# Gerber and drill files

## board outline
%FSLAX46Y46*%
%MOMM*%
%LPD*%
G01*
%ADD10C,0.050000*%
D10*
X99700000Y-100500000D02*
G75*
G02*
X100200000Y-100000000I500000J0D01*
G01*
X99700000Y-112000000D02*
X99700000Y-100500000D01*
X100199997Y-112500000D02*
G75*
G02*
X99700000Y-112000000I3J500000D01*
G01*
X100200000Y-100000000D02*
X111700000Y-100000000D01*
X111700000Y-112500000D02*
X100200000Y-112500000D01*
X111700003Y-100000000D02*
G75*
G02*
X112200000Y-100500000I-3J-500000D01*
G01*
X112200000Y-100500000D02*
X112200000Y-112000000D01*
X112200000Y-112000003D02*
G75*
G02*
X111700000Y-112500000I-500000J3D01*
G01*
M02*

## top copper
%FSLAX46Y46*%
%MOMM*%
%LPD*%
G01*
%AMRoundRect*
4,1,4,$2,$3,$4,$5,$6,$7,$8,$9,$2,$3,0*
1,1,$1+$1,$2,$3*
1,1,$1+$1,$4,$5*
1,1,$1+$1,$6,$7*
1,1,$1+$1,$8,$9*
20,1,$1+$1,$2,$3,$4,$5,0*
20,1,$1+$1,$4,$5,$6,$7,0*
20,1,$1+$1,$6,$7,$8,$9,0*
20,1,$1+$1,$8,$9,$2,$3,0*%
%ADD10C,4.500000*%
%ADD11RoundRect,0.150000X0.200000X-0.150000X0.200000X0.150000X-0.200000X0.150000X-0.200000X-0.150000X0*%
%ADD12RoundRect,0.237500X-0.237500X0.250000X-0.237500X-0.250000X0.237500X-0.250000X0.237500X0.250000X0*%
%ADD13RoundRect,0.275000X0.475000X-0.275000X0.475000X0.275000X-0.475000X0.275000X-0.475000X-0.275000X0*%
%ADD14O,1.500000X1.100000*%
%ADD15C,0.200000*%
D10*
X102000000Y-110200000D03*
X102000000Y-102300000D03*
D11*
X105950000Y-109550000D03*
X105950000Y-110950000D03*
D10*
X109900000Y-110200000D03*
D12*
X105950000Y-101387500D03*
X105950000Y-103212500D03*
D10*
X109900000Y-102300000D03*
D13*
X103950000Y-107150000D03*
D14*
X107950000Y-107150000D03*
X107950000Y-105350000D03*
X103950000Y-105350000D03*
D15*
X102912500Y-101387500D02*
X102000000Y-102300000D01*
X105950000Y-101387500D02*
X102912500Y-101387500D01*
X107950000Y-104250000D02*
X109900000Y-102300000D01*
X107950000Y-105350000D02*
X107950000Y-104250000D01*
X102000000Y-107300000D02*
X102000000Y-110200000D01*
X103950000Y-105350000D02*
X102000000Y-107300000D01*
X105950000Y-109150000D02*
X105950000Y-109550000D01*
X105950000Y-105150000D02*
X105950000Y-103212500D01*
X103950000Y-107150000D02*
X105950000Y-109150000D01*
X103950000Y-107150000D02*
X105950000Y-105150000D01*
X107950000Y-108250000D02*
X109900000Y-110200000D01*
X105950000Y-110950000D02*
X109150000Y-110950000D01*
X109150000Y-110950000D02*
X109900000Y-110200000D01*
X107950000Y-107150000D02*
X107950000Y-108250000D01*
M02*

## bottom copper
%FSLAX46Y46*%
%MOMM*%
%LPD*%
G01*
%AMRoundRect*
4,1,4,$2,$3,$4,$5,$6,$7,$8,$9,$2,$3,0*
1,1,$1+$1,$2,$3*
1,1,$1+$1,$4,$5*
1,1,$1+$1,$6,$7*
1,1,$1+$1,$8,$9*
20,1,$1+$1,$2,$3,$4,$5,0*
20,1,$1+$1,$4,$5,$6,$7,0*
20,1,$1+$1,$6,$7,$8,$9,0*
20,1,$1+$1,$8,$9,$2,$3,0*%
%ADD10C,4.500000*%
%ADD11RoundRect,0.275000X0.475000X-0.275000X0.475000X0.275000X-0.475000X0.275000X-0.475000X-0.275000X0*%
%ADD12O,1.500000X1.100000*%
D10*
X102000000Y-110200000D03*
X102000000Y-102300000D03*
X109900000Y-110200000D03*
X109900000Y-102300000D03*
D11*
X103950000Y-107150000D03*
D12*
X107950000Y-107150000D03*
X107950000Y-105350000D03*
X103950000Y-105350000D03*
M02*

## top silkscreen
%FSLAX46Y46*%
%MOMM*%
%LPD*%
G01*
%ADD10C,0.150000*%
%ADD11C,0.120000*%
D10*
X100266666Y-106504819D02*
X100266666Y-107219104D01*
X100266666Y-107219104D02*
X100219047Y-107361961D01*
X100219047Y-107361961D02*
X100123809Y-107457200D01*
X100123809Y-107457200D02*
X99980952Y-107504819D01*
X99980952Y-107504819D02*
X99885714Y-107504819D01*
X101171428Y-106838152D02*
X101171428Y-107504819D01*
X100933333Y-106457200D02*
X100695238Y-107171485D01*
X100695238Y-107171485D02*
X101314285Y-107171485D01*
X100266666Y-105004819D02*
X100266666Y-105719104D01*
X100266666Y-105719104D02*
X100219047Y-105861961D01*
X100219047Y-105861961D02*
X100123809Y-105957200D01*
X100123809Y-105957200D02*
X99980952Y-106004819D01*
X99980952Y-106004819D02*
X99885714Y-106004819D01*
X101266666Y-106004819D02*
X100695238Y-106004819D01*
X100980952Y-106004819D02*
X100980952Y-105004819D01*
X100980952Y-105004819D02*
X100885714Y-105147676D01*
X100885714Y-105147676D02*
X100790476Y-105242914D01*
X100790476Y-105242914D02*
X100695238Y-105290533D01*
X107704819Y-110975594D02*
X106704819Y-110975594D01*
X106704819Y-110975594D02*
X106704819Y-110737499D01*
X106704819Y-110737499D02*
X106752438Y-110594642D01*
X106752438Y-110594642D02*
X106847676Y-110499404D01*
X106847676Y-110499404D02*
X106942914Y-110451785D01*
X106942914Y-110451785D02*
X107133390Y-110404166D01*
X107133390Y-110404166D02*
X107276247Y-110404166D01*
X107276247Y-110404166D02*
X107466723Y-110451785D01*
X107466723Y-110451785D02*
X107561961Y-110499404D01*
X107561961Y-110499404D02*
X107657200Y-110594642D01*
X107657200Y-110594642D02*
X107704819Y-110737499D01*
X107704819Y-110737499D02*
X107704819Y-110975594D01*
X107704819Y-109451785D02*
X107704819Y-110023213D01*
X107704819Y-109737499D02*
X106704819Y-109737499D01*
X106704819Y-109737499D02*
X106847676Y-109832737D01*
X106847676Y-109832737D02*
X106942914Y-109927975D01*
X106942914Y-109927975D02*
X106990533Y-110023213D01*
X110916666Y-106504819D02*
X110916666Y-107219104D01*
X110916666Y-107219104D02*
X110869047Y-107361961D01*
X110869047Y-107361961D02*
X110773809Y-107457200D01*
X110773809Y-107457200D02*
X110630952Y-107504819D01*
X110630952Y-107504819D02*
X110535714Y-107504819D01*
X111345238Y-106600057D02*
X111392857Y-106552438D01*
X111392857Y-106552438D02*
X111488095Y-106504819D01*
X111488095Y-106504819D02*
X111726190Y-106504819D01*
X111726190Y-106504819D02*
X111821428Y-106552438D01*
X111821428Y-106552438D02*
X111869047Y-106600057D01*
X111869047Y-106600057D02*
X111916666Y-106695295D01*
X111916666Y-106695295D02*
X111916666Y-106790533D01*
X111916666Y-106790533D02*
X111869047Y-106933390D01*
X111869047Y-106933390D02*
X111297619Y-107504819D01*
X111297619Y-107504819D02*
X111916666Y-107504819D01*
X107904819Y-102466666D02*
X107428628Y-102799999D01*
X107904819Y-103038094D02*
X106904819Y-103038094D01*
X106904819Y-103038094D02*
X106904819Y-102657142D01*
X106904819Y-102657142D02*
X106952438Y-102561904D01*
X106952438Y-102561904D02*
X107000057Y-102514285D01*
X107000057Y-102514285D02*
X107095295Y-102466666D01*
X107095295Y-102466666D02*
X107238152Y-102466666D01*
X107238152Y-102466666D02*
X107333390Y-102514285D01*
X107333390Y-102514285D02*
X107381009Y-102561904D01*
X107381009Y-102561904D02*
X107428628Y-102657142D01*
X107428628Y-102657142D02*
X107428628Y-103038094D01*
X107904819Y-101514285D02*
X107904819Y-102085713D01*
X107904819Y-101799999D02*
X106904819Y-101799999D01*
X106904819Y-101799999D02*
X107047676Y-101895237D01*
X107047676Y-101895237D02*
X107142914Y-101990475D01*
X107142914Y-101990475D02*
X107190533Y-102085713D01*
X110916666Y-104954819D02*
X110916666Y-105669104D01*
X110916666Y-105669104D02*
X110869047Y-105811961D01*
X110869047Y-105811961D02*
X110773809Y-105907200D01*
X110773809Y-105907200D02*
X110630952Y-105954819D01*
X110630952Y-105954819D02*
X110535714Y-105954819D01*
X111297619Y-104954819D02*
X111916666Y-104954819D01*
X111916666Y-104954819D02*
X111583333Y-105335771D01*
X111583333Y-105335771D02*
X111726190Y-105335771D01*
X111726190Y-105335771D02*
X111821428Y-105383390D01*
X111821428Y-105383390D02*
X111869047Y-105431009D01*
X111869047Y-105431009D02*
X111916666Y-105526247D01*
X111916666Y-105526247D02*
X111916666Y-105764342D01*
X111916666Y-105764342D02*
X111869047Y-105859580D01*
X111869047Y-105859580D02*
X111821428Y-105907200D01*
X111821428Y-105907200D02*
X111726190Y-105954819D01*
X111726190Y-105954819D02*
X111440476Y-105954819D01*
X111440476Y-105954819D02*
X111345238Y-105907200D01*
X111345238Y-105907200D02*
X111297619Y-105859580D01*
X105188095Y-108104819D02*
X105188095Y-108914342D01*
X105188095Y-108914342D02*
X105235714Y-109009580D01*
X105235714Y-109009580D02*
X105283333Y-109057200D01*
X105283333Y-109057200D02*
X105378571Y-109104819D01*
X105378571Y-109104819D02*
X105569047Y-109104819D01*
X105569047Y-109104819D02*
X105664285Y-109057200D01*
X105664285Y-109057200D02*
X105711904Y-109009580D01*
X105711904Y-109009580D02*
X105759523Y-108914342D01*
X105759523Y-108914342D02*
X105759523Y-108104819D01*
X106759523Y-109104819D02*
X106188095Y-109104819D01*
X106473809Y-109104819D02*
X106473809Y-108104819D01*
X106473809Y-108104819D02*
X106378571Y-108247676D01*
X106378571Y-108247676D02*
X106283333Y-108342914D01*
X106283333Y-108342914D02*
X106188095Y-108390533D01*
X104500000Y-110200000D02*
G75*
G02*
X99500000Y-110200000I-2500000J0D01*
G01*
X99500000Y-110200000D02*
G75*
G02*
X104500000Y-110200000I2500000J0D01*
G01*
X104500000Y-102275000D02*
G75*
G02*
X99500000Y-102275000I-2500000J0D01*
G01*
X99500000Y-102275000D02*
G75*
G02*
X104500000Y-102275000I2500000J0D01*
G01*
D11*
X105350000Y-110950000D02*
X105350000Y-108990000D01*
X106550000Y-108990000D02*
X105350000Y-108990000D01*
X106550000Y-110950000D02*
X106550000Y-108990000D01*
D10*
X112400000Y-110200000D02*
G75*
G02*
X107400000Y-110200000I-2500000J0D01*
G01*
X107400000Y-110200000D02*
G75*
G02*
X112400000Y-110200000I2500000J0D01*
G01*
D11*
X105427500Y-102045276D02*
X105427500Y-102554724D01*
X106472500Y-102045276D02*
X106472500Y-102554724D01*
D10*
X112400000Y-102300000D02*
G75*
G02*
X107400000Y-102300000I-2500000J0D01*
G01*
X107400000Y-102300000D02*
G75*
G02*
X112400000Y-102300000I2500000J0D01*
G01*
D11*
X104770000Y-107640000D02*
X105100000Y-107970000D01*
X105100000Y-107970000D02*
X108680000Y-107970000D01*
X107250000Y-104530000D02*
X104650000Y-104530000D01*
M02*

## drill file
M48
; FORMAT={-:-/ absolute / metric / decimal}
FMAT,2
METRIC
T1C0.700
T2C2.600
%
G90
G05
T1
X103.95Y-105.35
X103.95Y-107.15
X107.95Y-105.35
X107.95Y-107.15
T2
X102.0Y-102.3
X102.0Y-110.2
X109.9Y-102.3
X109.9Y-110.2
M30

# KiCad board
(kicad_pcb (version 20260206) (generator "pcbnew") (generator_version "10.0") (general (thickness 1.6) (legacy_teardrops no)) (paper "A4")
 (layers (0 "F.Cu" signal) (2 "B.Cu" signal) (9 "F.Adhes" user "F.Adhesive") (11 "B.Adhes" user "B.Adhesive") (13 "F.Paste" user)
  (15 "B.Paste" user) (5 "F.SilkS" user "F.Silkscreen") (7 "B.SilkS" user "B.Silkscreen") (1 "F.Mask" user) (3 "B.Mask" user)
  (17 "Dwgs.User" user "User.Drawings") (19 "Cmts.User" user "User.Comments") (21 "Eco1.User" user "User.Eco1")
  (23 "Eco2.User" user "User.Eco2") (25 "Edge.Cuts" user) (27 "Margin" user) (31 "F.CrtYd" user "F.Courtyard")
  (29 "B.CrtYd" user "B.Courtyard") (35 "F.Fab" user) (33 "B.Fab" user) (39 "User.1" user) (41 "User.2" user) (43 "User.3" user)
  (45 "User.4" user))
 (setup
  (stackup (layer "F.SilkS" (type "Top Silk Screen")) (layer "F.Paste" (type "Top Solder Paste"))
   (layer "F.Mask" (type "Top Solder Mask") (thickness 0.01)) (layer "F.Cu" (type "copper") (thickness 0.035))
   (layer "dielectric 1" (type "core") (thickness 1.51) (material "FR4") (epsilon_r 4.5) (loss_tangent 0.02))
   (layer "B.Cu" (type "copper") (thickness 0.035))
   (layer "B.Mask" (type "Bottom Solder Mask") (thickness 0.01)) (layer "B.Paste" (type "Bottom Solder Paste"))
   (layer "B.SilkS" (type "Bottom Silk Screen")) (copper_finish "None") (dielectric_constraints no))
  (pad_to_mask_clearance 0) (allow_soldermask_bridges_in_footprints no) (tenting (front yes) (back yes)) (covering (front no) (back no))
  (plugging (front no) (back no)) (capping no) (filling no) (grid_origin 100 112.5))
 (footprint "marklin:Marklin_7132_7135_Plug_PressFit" (layer "F.Cu") (at 102 110.2)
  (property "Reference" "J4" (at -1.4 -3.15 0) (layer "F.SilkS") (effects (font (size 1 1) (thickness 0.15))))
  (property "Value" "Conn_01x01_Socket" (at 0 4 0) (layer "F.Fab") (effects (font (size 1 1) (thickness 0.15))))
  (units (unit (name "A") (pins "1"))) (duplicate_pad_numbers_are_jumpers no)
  (fp_circle (center 0 0) (end 2.5 0) (stroke (width 0.15) (type solid)) (fill no) (layer "F.SilkS"))
  (pad "1" thru_hole circle (at 0 0) (size 4.5 4.5) (drill 2.6) (layers "*.Cu" "*.Mask") (remove_unused_layers no) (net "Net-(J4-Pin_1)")))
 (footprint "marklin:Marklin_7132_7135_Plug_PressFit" (layer "F.Cu") (at 102 102.275)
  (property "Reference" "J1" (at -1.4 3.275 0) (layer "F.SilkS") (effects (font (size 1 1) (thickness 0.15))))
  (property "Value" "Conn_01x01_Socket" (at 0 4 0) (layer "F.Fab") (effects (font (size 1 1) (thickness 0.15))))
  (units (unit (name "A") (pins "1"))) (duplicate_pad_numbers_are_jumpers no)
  (fp_circle (center 0 0) (end 2.5 0) (stroke (width 0.15) (type solid)) (fill no) (layer "F.SilkS"))
  (pad "1" thru_hole circle (at 0 0.025) (size 4.5 4.5) (drill 2.6) (layers "*.Cu" "*.Mask") (remove_unused_layers no)
   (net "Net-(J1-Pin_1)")))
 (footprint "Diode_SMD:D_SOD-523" (layer "F.Cu") (at 105.95 110.25 -90)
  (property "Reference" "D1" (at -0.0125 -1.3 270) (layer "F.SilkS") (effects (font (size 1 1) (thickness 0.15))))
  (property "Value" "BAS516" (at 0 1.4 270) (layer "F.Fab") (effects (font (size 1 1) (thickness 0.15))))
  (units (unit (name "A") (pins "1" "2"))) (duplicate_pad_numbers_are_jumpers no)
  (fp_line (start 0.7 0.6) (end -1.26 0.6) (stroke (width 0.12) (type solid)) (layer "F.SilkS"))
  (fp_line (start -1.26 -0.6) (end -1.26 0.6) (stroke (width 0.12) (type solid)) (layer "F.SilkS"))
  (fp_line (start 0.7 -0.6) (end -1.26 -0.6) (stroke (width 0.12) (type solid)) (layer "F.SilkS"))
  (pad "1" smd roundrect (at -0.7 0 90) (size 0.6 0.7) (layers "F.Cu" "F.Mask" "F.Paste") (roundrect_rratio 0.25) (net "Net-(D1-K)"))
  (pad "2" smd roundrect (at 0.7 0 90) (size 0.6 0.7) (layers "F.Cu" "F.Mask" "F.Paste") (roundrect_rratio 0.25) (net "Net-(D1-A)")))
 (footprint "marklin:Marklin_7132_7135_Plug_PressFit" (layer "F.Cu") (at 109.9 110.2 -90)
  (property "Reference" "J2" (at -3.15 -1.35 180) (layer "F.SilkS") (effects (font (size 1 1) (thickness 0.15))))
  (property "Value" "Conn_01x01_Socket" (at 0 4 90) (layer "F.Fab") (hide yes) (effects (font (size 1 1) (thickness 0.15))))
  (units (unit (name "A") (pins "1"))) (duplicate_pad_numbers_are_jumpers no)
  (fp_circle (center 0 0) (end 2.5 0) (stroke (width 0.15) (type solid)) (fill no) (layer "F.SilkS"))
  (pad "1" thru_hole circle (at 0 0 270) (size 4.5 4.5) (drill 2.6) (layers "*.Cu" "*.Mask") (remove_unused_layers no) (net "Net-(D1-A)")))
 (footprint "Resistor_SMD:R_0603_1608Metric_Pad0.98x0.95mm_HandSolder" (layer "F.Cu") (at 105.95 102.3 -90)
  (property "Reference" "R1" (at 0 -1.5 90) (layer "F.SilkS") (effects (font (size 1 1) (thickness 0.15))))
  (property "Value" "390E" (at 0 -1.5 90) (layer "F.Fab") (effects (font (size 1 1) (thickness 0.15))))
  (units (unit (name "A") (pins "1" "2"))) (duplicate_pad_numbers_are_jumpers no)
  (fp_line (start -0.254724 0.5225) (end 0.254724 0.5225) (stroke (width 0.12) (type solid)) (layer "F.SilkS"))
  (fp_line (start -0.254724 -0.5225) (end 0.254724 -0.5225) (stroke (width 0.12) (type solid)) (layer "F.SilkS"))
  (pad "1" smd roundrect (at -0.9125 0 270) (size 0.975 0.95) (layers "F.Cu" "F.Mask" "F.Paste") (roundrect_rratio 0.25)
   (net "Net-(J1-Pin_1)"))
  (pad "2" smd roundrect (at 0.9125 0 270) (size 0.975 0.95) (layers "F.Cu" "F.Mask" "F.Paste") (roundrect_rratio 0.25) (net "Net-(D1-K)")))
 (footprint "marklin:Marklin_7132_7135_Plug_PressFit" (layer "F.Cu") (at 109.9 102.3)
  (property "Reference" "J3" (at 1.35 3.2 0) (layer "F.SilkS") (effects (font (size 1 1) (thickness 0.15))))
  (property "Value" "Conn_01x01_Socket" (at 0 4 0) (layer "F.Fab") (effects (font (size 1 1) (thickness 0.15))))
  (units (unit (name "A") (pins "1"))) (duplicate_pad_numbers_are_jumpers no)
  (fp_circle (center 0 0) (end 2.5 0) (stroke (width 0.15) (type solid)) (fill no) (layer "F.SilkS"))
  (pad "1" thru_hole circle (at 0 0) (size 4.5 4.5) (drill 2.6) (layers "*.Cu" "*.Mask") (remove_unused_layers no) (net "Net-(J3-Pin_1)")))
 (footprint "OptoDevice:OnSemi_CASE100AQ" (layer "F.Cu") (at 103.95 107.15 90)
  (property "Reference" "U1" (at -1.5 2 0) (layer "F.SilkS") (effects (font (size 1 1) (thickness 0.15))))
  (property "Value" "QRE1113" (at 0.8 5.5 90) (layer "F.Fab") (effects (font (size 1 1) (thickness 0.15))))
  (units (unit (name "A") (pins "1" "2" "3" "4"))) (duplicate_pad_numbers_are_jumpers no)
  (fp_line (start -0.49 0.82) (end -0.82 1.15) (stroke (width 0.12) (type solid)) (layer "F.SilkS"))
  (fp_line (start -0.82 1.15) (end -0.82 4.73) (stroke (width 0.12) (type solid)) (layer "F.SilkS"))
  (fp_line (start 2.62 3.3) (end 2.62 0.7) (stroke (width 0.12) (type solid)) (layer "F.SilkS"))
  (pad "1" thru_hole roundrect (at 0 0 90) (size 1.1 1.5) (drill 0.7) (layers "*.Cu" "*.Mask") (remove_unused_layers no)
   (roundrect_rratio 0.25) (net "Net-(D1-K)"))
  (pad "2" thru_hole oval (at 0 4 90) (size 1.1 1.5) (drill 0.7) (layers "*.Cu" "*.Mask") (remove_unused_layers no) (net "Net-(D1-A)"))
  (pad "3" thru_hole oval (at 1.8 4 90) (size 1.1 1.5) (drill 0.7) (layers "*.Cu" "*.Mask") (remove_unused_layers no) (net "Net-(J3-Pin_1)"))
  (pad "4" thru_hole oval (at 1.8 0 90) (size 1.1 1.5) (drill 0.7) (layers "*.Cu" "*.Mask") (remove_unused_layers no) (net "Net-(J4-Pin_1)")))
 (gr_arc (start 99.7 100.5) (mid 99.846447 100.146447) (end 100.2 100) (stroke (width 0.05) (type solid)) (layer "Edge.Cuts"))
 (gr_line (start 99.7 112) (end 99.7 100.5) (stroke (width 0.05) (type default)) (layer "Edge.Cuts"))
 (gr_arc (start 100.199997 112.5) (mid 99.846446 112.353552) (end 99.7 112) (stroke (width 0.05) (type solid)) (layer "Edge.Cuts"))
 (gr_line (start 100.2 100) (end 111.7 100) (stroke (width 0.05) (type solid)) (layer "Edge.Cuts"))
 (gr_line (start 111.7 112.5) (end 100.2 112.5) (stroke (width 0.05) (type solid)) (layer "Edge.Cuts"))
 (gr_arc (start 111.700003 100) (mid 112.053554 100.146448) (end 112.2 100.5) (stroke (width 0.05) (type solid)) (layer "Edge.Cuts"))
 (gr_line (start 112.2 100.5) (end 112.2 112) (stroke (width 0.05) (type solid)) (layer "Edge.Cuts"))
 (gr_arc (start 112.2 112.000003) (mid 112.053552 112.353554) (end 111.7 112.5) (stroke (width 0.05) (type solid)) (layer "Edge.Cuts"))
 (segment (start 102.9125 101.3875) (end 102 102.3) (width 0.2) (layer "F.Cu") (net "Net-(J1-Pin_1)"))
 (segment (start 105.95 101.3875) (end 102.9125 101.3875) (width 0.2) (layer "F.Cu") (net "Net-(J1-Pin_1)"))
 (segment (start 107.95 104.25) (end 109.9 102.3) (width 0.2) (layer "F.Cu") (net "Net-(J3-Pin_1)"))
 (segment (start 107.95 105.35) (end 107.95 104.25) (width 0.2) (layer "F.Cu") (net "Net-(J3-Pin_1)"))
 (segment (start 102 107.3) (end 102 110.2) (width 0.2) (layer "F.Cu") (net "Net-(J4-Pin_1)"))
 (segment (start 103.95 105.35) (end 102 107.3) (width 0.2) (layer "F.Cu") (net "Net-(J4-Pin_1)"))
 (segment (start 105.95 109.15) (end 105.95 109.55) (width 0.2) (layer "F.Cu") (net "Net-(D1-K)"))
 (segment (start 105.95 105.15) (end 105.95 103.2125) (width 0.2) (layer "F.Cu") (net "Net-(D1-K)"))
 (segment (start 103.95 107.15) (end 105.95 109.15) (width 0.2) (layer "F.Cu") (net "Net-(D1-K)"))
 (segment (start 103.95 107.15) (end 105.95 105.15) (width 0.2) (layer "F.Cu") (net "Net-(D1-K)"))
 (segment (start 107.95 108.25) (end 109.9 110.2) (width 0.2) (layer "F.Cu") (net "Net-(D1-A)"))
 (segment (start 105.95 110.95) (end 109.15 110.95) (width 0.2) (layer "F.Cu") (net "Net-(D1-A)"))
 (segment (start 109.15 110.95) (end 109.9 110.2) (width 0.2) (layer "F.Cu") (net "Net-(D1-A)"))
 (segment (start 107.95 107.15) (end 107.95 108.25) (width 0.2) (layer "F.Cu") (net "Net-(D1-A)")))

